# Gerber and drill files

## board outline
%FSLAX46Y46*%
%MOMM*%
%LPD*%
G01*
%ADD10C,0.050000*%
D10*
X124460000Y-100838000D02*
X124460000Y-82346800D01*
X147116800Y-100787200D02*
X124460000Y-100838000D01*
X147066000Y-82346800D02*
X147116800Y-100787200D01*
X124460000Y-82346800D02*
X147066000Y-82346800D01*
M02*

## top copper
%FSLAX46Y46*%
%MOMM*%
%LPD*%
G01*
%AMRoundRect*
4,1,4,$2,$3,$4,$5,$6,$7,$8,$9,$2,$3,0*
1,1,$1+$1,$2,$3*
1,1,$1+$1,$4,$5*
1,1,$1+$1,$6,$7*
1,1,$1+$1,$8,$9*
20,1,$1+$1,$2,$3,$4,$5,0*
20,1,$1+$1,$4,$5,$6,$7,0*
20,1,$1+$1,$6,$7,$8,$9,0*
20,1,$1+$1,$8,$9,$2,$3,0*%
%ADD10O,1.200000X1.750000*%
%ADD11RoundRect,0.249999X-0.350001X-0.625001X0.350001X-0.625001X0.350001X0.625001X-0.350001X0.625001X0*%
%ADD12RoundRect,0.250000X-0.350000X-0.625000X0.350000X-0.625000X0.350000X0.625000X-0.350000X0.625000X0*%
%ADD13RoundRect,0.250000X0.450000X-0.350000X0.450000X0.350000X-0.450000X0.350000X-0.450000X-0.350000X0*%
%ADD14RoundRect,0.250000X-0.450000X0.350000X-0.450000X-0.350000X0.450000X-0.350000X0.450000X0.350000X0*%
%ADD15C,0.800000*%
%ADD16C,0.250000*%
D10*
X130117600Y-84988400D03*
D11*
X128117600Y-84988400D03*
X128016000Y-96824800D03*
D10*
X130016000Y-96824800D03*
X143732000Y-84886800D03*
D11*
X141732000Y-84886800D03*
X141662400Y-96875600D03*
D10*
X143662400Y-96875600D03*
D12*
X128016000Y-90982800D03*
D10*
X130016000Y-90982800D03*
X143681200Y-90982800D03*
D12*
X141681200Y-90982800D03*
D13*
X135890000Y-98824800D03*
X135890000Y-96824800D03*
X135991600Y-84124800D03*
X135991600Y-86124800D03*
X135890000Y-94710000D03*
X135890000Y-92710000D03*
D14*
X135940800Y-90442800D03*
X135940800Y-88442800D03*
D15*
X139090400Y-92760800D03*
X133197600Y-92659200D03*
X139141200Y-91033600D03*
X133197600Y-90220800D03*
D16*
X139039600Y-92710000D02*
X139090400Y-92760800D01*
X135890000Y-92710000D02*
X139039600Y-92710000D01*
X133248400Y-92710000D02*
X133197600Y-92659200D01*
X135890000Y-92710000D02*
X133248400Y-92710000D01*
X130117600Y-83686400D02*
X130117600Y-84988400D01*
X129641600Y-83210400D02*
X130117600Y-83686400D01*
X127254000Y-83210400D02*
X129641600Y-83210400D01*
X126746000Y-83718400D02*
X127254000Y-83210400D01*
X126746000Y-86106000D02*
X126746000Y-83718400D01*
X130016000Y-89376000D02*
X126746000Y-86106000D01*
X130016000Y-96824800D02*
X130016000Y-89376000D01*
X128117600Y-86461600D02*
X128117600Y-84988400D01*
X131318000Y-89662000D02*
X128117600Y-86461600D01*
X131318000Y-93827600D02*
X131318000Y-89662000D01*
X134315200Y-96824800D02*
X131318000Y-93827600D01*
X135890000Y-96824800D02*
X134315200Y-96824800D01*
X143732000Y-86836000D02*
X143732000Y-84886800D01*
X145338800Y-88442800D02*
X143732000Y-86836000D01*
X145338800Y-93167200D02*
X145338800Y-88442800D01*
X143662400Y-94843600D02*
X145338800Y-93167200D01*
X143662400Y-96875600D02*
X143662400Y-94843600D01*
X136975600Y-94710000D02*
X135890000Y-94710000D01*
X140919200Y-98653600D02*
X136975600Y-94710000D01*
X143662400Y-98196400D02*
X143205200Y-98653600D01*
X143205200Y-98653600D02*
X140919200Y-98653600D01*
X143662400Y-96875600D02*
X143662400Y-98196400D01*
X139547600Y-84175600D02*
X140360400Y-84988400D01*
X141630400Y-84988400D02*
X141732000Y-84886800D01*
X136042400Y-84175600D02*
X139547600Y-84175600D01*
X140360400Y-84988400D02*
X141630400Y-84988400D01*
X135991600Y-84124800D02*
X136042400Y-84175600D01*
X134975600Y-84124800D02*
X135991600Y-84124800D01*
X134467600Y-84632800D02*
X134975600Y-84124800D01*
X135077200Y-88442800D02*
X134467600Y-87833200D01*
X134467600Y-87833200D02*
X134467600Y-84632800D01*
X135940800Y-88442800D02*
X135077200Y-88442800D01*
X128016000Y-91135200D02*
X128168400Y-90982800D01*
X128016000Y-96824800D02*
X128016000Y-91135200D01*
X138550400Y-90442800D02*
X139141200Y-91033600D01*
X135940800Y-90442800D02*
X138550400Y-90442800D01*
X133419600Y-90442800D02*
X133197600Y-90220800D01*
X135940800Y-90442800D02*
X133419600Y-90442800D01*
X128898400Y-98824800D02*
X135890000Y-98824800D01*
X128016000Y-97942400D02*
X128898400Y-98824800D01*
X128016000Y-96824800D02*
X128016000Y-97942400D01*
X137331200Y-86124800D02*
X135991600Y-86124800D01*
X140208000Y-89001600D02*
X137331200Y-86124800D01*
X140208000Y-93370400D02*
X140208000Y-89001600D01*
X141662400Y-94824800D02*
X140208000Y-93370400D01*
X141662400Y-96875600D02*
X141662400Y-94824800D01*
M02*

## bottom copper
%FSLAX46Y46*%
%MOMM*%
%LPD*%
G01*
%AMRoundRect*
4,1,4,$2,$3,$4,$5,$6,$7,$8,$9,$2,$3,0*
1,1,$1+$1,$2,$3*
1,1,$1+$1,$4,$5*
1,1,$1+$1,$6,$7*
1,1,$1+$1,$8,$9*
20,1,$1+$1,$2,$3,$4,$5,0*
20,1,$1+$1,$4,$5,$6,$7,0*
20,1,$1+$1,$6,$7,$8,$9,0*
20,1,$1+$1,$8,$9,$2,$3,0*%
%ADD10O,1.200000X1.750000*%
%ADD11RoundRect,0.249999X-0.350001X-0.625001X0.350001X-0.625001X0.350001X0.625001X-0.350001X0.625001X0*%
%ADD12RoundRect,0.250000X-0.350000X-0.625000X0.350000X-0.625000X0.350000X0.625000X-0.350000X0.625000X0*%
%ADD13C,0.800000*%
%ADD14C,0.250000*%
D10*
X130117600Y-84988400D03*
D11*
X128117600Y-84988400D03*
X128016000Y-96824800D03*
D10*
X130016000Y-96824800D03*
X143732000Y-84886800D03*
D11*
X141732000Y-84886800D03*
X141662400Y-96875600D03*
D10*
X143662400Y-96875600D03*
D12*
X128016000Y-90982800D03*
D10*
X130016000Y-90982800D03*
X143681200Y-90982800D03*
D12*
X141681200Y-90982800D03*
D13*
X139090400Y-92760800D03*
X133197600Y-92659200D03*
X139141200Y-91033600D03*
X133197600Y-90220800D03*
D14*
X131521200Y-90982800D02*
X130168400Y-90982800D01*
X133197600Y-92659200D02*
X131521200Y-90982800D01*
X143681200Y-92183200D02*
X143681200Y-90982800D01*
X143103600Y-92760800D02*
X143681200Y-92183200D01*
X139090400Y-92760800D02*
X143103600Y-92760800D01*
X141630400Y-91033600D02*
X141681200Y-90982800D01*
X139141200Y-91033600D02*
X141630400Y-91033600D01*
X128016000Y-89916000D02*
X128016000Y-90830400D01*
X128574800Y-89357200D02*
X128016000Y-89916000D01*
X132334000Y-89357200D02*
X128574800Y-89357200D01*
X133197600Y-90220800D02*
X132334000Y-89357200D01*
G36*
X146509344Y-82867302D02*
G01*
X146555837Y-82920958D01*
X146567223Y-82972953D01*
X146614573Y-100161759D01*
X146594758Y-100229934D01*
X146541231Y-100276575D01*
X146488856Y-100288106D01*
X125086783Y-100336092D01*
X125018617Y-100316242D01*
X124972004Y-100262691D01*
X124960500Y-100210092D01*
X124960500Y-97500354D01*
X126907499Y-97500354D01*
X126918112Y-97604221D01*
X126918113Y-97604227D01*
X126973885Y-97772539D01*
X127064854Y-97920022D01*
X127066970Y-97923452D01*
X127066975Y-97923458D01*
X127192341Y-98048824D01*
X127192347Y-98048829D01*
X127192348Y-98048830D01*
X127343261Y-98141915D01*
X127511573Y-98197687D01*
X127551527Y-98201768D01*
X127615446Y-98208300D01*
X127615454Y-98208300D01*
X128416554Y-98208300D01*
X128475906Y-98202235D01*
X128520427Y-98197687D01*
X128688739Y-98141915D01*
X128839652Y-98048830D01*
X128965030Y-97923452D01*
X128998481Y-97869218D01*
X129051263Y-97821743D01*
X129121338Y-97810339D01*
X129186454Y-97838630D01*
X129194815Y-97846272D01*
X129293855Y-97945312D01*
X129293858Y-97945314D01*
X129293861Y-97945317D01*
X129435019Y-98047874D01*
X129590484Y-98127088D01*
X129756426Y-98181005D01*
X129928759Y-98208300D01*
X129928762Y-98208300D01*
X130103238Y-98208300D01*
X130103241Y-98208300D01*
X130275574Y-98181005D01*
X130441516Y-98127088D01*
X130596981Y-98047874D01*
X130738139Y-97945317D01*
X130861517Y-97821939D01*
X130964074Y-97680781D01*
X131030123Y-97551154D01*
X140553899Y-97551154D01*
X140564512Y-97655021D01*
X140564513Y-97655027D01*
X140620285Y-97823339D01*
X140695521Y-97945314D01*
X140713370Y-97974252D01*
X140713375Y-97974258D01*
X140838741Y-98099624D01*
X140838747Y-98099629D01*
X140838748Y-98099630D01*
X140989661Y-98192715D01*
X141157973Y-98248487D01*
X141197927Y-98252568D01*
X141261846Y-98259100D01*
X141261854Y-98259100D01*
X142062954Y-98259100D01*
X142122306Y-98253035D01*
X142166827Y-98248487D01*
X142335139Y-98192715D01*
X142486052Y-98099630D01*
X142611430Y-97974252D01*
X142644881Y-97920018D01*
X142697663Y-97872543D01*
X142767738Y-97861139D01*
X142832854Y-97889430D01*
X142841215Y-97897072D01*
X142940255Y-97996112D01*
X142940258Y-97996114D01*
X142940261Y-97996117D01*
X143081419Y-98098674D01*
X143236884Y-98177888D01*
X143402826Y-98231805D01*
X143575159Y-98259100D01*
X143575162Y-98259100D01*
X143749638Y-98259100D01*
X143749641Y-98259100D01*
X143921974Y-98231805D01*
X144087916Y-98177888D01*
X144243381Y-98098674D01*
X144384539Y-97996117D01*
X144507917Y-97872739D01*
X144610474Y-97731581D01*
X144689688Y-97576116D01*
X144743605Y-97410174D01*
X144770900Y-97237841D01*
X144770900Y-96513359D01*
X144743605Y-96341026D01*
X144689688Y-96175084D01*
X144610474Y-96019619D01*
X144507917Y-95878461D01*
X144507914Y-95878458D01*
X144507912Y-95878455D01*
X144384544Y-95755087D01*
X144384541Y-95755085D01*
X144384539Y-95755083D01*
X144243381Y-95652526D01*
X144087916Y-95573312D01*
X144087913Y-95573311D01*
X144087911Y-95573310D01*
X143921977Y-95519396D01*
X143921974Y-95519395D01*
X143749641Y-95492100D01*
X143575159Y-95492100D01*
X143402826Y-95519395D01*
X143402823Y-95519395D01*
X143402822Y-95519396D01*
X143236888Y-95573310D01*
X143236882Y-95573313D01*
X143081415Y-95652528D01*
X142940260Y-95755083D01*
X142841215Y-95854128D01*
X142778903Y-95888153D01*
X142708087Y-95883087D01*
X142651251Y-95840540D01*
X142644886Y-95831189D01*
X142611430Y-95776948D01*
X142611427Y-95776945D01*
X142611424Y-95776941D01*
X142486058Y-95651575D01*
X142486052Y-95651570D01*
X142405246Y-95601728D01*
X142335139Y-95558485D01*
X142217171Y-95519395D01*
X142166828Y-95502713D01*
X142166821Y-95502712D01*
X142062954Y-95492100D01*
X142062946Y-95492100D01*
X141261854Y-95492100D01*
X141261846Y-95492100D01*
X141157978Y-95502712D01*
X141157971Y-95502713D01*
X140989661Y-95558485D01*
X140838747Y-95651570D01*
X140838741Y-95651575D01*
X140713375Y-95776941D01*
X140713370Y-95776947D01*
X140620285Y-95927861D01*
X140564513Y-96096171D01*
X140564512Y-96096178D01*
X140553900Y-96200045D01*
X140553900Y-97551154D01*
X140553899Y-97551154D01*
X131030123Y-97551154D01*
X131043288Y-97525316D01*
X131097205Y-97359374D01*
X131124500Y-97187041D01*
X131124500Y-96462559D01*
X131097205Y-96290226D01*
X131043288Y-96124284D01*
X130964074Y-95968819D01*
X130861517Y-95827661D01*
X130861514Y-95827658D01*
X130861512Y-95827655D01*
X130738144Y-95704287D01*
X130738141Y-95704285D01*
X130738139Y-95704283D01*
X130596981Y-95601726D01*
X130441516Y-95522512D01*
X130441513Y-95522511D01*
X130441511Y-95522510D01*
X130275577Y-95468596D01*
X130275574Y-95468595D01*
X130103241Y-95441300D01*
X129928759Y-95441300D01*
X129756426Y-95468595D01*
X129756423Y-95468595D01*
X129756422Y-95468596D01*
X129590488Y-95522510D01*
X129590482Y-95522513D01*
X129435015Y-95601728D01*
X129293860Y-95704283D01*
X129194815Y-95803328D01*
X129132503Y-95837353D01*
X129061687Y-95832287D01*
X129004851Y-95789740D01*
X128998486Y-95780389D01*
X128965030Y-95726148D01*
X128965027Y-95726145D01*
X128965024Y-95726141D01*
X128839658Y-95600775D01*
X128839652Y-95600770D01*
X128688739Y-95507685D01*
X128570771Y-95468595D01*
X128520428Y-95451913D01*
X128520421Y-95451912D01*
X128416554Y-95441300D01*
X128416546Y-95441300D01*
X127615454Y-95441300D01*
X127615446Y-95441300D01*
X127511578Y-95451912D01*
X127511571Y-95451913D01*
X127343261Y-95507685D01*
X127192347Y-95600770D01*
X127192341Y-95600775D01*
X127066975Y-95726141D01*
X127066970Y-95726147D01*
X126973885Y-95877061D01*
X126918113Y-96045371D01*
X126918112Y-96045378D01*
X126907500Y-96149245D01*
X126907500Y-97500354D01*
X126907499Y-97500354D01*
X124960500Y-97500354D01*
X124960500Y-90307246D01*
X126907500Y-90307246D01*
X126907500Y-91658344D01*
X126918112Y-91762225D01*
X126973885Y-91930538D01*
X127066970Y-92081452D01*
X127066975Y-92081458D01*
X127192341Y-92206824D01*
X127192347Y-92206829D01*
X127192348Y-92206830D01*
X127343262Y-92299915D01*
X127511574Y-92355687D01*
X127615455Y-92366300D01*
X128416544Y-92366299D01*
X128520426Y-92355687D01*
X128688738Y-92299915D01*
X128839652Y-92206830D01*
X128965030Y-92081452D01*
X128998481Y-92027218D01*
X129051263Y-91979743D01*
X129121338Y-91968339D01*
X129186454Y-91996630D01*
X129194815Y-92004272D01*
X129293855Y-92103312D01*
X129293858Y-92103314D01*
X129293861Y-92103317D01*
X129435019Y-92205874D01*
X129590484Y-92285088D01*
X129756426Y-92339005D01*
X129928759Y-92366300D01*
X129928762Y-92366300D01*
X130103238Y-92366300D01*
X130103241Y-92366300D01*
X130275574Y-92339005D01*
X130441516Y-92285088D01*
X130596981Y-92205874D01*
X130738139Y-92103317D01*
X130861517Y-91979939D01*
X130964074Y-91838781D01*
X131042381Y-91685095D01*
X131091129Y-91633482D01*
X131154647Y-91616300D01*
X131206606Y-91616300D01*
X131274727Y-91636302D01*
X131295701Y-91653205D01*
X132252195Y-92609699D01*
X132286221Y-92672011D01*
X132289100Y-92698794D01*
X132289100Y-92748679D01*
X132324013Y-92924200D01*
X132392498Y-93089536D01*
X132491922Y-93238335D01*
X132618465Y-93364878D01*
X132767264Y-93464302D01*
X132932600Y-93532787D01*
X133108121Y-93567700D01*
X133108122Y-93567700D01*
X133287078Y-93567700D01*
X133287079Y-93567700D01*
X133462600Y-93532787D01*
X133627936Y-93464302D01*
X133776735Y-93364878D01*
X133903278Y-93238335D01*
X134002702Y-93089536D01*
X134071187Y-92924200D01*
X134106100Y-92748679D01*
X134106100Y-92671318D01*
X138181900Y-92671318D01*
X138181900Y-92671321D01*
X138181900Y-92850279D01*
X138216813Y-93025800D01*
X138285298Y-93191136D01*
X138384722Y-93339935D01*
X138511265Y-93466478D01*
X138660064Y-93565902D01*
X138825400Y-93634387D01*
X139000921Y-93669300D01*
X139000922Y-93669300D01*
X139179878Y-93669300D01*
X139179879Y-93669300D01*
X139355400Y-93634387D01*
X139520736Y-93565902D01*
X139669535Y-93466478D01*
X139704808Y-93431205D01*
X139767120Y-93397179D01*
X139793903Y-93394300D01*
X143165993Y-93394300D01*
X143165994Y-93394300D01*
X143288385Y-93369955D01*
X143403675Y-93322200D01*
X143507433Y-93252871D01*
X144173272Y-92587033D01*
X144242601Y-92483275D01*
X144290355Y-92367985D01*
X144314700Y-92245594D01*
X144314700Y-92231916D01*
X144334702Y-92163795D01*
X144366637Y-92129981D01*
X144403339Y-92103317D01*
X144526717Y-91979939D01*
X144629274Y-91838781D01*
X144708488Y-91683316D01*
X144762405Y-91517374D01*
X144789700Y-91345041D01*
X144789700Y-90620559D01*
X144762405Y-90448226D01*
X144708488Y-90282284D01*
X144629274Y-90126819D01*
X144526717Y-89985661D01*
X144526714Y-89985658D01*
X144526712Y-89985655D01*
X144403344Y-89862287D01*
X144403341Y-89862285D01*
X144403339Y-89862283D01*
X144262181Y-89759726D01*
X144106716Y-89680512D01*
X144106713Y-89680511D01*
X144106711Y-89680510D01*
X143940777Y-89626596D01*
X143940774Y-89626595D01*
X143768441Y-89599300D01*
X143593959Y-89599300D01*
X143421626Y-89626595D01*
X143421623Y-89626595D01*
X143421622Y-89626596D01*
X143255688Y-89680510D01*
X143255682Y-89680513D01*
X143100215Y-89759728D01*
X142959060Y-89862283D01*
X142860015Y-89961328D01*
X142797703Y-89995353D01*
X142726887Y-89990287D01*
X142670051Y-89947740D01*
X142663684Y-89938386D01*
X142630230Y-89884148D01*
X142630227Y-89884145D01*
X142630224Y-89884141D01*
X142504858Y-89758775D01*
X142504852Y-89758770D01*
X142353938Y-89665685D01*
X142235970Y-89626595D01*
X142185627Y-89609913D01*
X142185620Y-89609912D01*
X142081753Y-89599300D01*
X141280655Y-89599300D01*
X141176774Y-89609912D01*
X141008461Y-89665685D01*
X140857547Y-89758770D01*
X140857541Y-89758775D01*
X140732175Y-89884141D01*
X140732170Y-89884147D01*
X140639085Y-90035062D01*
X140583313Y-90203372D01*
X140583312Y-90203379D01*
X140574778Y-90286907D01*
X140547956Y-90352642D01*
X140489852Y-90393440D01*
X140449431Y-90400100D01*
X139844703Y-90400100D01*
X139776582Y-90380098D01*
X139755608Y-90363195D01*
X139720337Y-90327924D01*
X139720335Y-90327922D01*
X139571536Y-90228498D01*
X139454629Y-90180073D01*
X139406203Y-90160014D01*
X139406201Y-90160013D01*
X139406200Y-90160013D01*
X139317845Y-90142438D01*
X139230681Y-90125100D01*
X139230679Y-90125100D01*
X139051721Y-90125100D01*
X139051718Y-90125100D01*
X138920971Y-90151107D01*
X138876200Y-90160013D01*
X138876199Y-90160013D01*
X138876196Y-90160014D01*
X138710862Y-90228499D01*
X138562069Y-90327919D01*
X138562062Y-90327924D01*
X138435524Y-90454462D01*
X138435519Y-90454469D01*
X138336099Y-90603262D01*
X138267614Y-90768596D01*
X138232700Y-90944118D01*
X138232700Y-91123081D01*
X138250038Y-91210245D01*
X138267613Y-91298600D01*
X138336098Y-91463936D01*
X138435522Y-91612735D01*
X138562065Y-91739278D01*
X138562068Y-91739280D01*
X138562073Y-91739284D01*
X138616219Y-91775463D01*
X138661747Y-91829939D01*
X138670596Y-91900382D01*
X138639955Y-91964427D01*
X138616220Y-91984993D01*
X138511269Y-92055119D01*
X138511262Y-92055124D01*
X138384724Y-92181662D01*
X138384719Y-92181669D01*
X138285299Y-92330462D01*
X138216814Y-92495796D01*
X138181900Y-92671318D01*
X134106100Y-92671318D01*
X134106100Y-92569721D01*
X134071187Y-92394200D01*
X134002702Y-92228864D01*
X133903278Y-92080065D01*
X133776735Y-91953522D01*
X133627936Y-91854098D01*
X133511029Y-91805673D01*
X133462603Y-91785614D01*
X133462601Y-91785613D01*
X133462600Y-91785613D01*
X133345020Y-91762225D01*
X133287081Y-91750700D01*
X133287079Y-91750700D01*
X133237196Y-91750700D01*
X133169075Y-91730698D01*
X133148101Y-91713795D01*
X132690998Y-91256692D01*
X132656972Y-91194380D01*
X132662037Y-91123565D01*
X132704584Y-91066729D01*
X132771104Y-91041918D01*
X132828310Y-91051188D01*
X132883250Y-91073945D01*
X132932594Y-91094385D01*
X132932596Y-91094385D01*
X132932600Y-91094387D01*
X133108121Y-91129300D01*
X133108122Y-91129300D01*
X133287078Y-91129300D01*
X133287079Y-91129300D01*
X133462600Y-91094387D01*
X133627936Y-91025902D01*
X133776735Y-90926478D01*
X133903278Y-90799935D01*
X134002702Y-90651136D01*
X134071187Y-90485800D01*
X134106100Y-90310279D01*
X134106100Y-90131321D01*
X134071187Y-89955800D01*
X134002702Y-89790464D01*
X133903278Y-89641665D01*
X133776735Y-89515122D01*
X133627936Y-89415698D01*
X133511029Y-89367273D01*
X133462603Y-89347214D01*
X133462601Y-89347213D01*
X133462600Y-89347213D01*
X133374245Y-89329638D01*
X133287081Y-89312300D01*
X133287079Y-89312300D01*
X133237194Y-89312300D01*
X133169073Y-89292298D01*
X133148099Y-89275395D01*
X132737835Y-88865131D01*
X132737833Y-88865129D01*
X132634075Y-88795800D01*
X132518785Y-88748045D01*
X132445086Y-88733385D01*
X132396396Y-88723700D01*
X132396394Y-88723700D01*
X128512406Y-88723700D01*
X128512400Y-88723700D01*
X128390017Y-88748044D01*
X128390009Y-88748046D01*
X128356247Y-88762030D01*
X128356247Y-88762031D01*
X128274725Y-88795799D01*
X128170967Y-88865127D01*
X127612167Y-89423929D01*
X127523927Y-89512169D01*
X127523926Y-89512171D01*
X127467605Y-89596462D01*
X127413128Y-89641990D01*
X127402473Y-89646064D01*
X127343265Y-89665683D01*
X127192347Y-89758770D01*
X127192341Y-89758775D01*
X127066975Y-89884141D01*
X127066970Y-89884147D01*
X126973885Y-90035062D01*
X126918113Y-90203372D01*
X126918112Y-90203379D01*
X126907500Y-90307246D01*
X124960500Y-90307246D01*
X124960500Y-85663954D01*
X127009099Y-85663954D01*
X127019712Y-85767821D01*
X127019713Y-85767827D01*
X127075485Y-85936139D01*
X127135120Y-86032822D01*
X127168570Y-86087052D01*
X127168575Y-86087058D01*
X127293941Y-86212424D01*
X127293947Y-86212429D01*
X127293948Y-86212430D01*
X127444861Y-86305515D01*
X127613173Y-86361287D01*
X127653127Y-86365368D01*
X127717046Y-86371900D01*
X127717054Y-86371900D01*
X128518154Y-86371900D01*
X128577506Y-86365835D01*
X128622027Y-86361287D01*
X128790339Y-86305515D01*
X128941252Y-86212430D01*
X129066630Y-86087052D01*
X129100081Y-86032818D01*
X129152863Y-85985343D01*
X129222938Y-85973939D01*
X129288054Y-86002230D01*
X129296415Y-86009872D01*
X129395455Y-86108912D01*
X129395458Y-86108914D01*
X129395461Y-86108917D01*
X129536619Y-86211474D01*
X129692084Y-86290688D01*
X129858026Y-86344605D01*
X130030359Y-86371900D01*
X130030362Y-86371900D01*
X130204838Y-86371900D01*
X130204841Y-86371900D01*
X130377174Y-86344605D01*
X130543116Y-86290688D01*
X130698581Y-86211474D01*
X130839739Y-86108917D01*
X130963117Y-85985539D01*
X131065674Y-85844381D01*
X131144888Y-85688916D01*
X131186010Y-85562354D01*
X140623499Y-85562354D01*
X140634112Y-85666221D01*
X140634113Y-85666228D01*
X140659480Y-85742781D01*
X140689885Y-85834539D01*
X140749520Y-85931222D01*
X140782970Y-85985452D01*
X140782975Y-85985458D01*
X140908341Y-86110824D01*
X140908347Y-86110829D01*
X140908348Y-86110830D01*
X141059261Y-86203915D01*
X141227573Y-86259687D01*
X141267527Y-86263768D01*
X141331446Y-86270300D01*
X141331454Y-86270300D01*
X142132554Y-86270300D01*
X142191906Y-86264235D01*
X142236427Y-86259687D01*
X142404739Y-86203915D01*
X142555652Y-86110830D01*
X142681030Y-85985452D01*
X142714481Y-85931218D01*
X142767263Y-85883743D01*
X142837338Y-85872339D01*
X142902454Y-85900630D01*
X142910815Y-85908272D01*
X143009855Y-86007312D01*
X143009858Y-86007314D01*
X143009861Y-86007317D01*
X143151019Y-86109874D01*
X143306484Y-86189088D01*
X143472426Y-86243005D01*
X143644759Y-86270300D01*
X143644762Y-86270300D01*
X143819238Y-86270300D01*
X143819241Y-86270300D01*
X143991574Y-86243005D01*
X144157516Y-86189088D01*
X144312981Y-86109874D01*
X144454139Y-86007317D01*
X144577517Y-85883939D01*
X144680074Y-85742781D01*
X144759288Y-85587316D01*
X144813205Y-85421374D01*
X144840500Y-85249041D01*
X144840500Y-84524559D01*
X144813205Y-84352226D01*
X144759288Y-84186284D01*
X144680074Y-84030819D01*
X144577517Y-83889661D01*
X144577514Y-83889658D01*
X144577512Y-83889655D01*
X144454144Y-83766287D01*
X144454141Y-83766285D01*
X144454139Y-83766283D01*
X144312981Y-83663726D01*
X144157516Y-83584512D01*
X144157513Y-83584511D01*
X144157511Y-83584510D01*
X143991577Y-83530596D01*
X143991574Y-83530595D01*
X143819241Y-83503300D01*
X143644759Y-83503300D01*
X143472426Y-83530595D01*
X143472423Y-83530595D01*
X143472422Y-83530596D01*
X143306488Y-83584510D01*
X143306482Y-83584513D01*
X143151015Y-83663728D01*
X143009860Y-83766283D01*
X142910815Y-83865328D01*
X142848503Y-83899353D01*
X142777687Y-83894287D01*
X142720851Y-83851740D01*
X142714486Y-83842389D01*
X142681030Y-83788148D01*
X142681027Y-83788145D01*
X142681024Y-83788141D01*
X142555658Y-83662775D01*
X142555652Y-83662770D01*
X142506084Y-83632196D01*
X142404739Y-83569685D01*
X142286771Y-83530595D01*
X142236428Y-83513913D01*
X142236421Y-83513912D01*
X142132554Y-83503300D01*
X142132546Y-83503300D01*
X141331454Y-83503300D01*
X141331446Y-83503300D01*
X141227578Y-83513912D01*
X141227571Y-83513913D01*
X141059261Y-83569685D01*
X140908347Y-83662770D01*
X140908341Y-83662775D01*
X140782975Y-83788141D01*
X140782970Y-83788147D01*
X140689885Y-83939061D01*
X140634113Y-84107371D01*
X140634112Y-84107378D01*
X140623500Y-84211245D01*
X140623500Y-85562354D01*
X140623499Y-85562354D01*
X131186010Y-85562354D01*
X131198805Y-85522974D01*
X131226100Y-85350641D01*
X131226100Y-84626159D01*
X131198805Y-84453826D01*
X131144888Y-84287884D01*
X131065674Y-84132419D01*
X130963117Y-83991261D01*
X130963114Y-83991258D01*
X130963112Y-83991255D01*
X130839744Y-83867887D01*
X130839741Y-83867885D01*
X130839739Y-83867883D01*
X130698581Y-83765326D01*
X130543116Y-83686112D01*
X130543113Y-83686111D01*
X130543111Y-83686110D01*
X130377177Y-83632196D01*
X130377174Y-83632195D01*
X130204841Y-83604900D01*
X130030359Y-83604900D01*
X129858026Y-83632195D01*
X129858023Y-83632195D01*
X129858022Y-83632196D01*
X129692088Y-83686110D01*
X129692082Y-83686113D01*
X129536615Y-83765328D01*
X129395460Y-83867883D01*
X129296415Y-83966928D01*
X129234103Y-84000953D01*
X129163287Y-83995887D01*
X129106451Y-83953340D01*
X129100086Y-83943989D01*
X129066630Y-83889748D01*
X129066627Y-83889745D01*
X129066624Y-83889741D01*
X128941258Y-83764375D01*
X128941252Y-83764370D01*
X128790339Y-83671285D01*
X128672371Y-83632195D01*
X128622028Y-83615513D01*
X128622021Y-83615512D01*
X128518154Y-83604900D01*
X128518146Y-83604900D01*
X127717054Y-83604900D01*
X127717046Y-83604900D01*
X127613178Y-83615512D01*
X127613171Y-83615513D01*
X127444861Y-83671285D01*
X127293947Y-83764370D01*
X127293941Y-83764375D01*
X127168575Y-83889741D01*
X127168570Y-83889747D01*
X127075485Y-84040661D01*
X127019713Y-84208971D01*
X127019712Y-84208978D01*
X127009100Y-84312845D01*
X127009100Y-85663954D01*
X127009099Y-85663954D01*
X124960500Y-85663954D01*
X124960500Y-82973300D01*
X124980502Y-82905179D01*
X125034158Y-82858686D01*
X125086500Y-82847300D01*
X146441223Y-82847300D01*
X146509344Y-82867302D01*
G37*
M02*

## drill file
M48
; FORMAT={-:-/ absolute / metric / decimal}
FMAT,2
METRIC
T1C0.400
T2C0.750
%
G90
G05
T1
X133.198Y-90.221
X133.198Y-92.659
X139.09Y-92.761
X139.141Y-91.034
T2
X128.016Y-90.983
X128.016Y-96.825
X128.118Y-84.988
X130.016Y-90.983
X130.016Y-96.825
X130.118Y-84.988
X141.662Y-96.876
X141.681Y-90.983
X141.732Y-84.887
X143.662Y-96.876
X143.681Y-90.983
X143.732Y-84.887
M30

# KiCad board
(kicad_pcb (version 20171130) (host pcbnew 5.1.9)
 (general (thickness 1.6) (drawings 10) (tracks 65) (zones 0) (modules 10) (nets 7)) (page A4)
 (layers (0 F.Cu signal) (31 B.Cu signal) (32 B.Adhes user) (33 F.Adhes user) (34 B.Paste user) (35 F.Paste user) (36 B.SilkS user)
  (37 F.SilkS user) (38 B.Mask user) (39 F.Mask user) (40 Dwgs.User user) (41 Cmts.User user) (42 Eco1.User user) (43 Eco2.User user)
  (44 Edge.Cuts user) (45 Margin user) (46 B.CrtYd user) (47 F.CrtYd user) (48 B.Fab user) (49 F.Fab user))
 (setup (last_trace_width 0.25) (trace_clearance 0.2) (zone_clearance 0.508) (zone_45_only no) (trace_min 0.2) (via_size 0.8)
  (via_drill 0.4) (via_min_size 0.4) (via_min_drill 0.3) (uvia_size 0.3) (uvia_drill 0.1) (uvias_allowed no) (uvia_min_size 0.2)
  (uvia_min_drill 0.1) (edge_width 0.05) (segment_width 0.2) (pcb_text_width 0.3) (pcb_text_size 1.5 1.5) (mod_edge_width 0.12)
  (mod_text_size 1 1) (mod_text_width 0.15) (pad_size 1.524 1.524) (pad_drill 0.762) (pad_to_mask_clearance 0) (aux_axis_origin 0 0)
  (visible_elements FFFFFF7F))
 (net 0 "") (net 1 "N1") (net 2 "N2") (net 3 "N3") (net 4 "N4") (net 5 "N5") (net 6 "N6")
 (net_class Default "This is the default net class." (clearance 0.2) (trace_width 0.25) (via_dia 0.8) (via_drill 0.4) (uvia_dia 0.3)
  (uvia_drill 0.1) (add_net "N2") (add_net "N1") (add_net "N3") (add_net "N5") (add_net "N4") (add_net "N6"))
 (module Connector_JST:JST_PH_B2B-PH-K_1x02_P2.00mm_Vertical (layer F.Cu) (at 128.1176 84.9884)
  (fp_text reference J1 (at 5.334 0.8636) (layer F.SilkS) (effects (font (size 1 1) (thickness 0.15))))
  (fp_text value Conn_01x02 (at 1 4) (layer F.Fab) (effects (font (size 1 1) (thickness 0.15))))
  (pad 2 thru_hole oval (at 2 0) (size 1.2 1.75) (drill 0.75) (layers *.Cu *.Mask) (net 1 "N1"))
  (pad 1 thru_hole roundrect (at 0 0) (size 1.2 1.75) (drill 0.75) (layers *.Cu *.Mask) (roundrect_rratio 0.2083325) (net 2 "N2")))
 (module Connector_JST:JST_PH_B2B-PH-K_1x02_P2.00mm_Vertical (layer F.Cu) (at 128.016 96.8248)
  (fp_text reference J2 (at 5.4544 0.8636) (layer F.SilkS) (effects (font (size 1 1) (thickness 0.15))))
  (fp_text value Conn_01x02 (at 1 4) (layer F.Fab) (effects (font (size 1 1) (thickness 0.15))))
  (pad 1 thru_hole roundrect (at 0 0) (size 1.2 1.75) (drill 0.75) (layers *.Cu *.Mask) (roundrect_rratio 0.2083325) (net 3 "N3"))
  (pad 2 thru_hole oval (at 2 0) (size 1.2 1.75) (drill 0.75) (layers *.Cu *.Mask) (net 1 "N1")))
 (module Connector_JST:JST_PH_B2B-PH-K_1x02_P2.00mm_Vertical (layer F.Cu) (at 141.732 84.8868)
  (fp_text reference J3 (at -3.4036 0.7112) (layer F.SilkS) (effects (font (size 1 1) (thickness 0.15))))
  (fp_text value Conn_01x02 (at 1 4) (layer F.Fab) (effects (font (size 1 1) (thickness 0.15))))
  (pad 2 thru_hole oval (at 2 0) (size 1.2 1.75) (drill 0.75) (layers *.Cu *.Mask) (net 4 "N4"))
  (pad 1 thru_hole roundrect (at 0 0) (size 1.2 1.75) (drill 0.75) (layers *.Cu *.Mask) (roundrect_rratio 0.2083325) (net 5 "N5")))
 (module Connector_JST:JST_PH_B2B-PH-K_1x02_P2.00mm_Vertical (layer F.Cu) (at 141.6624 96.8756)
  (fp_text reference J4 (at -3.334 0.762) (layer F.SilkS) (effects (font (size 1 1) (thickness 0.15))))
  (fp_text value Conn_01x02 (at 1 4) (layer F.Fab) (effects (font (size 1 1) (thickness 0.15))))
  (pad 1 thru_hole roundrect (at 0 0) (size 1.2 1.75) (drill 0.75) (layers *.Cu *.Mask) (roundrect_rratio 0.2083325) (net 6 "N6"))
  (pad 2 thru_hole oval (at 2 0) (size 1.2 1.75) (drill 0.75) (layers *.Cu *.Mask) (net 4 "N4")))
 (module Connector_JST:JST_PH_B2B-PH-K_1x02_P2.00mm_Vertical (layer F.Cu) (at 128.016 90.9828)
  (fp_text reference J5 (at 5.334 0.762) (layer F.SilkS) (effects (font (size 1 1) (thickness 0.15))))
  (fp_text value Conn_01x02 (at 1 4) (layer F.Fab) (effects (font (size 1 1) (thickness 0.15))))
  (pad 1 thru_hole roundrect (at 0 0) (size 1.2 1.75) (drill 0.75) (layers *.Cu *.Mask) (roundrect_rratio 0.208333) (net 3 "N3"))
  (pad 2 thru_hole oval (at 2 0) (size 1.2 1.75) (drill 0.75) (layers *.Cu *.Mask) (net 1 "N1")))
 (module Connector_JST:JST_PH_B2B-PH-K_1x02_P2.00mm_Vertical (layer F.Cu) (at 141.6812 90.9828)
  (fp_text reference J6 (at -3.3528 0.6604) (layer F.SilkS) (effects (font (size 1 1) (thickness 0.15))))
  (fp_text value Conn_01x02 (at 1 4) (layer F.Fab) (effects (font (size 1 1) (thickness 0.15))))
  (pad 2 thru_hole oval (at 2 0) (size 1.2 1.75) (drill 0.75) (layers *.Cu *.Mask) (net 1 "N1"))
  (pad 1 thru_hole roundrect (at 0 0) (size 1.2 1.75) (drill 0.75) (layers *.Cu *.Mask) (roundrect_rratio 0.208333) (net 3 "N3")))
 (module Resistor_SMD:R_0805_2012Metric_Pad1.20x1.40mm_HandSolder (layer F.Cu) (at 135.89 97.8248 90)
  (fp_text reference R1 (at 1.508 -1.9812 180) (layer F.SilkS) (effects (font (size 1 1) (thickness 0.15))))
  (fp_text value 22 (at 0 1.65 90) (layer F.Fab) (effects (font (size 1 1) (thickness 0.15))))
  (pad 1 smd roundrect (at -1 0 90) (size 1.2 1.4) (layers F.Cu F.Paste F.Mask) (roundrect_rratio 0.208333) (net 3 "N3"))
  (pad 2 smd roundrect (at 1 0 90) (size 1.2 1.4) (layers F.Cu F.Paste F.Mask) (roundrect_rratio 0.208333) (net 2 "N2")))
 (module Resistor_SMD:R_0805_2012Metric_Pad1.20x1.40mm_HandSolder (layer F.Cu) (at 135.9916 85.1248 90)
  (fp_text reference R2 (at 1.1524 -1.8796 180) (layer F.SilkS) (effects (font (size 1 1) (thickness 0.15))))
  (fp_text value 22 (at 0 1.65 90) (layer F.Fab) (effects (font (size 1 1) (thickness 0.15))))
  (pad 2 smd roundrect (at 1 0 90) (size 1.2 1.4) (layers F.Cu F.Paste F.Mask) (roundrect_rratio 0.208333) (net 5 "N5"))
  (pad 1 smd roundrect (at -1 0 90) (size 1.2 1.4) (layers F.Cu F.Paste F.Mask) (roundrect_rratio 0.208333) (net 6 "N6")))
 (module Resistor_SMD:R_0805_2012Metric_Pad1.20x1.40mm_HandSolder (layer F.Cu) (at 135.89 93.71 90)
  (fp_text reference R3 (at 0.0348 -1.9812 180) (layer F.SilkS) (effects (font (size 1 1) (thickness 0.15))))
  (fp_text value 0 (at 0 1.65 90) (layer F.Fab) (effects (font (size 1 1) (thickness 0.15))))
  (pad 1 smd roundrect (at -1 0 90) (size 1.2 1.4) (layers F.Cu F.Paste F.Mask) (roundrect_rratio 0.208333) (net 4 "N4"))
  (pad 2 smd roundrect (at 1 0 90) (size 1.2 1.4) (layers F.Cu F.Paste F.Mask) (roundrect_rratio 0.208333) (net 1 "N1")))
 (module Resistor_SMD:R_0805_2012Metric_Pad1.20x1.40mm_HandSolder (layer F.Cu) (at 135.9408 89.4428 270)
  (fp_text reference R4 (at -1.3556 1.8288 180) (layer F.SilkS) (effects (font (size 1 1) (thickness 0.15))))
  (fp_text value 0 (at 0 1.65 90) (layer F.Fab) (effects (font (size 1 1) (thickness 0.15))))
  (pad 2 smd roundrect (at 1 0 270) (size 1.2 1.4) (layers F.Cu F.Paste F.Mask) (roundrect_rratio 0.208333) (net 3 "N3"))
  (pad 1 smd roundrect (at -1 0 270) (size 1.2 1.4) (layers F.Cu F.Paste F.Mask) (roundrect_rratio 0.208333) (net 5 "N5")))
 (gr_line (start 124.46 100.838) (end 124.46 82.3468) (layer Edge.Cuts) (width 0.05))
 (gr_line (start 147.1168 100.7872) (end 124.46 100.838) (layer Edge.Cuts) (width 0.05))
 (gr_line (start 147.066 82.3468) (end 147.1168 100.7872) (layer Edge.Cuts) (width 0.05))
 (gr_line (start 124.46 82.3468) (end 147.066 82.3468) (layer Edge.Cuts) (width 0.05))
 (via (at 139.0904 92.7608) (size 0.8) (drill 0.4) (layers F.Cu B.Cu) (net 1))
 (segment (start 139.0396 92.71) (end 139.0904 92.7608) (width 0.25) (layer F.Cu) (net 1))
 (segment (start 135.89 92.71) (end 139.0396 92.71) (width 0.25) (layer F.Cu) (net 1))
 (via (at 133.1976 92.6592) (size 0.8) (drill 0.4) (layers F.Cu B.Cu) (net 1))
 (segment (start 133.2484 92.71) (end 133.1976 92.6592) (width 0.25) (layer F.Cu) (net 1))
 (segment (start 135.89 92.71) (end 133.2484 92.71) (width 0.25) (layer F.Cu) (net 1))
 (segment (start 131.5212 90.9828) (end 130.1684 90.9828) (width 0.25) (layer B.Cu) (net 1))
 (segment (start 133.1976 92.6592) (end 131.5212 90.9828) (width 0.25) (layer B.Cu) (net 1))
 (segment (start 130.1176 83.6864) (end 130.1176 84.9884) (width 0.25) (layer F.Cu) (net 1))
 (segment (start 129.6416 83.2104) (end 130.1176 83.6864) (width 0.25) (layer F.Cu) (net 1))
 (segment (start 127.254 83.2104) (end 129.6416 83.2104) (width 0.25) (layer F.Cu) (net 1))
 (segment (start 126.746 83.7184) (end 127.254 83.2104) (width 0.25) (layer F.Cu) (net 1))
 (segment (start 126.746 86.106) (end 126.746 83.7184) (width 0.25) (layer F.Cu) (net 1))
 (segment (start 130.016 89.376) (end 126.746 86.106) (width 0.25) (layer F.Cu) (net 1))
 (segment (start 130.016 96.8248) (end 130.016 89.376) (width 0.25) (layer F.Cu) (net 1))
 (segment (start 143.6812 92.1832) (end 143.6812 90.9828) (width 0.25) (layer B.Cu) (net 1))
 (segment (start 143.1036 92.7608) (end 143.6812 92.1832) (width 0.25) (layer B.Cu) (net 1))
 (segment (start 139.0904 92.7608) (end 143.1036 92.7608) (width 0.25) (layer B.Cu) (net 1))
 (segment (start 128.1176 86.4616) (end 128.1176 84.9884) (width 0.25) (layer F.Cu) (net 2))
 (segment (start 131.318 89.662) (end 128.1176 86.4616) (width 0.25) (layer F.Cu) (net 2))
 (segment (start 131.318 93.8276) (end 131.318 89.662) (width 0.25) (layer F.Cu) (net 2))
 (segment (start 134.3152 96.8248) (end 131.318 93.8276) (width 0.25) (layer F.Cu) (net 2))
 (segment (start 135.89 96.8248) (end 134.3152 96.8248) (width 0.25) (layer F.Cu) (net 2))
 (segment (start 143.732 86.836) (end 143.732 84.8868) (width 0.25) (layer F.Cu) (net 4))
 (segment (start 145.3388 88.4428) (end 143.732 86.836) (width 0.25) (layer F.Cu) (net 4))
 (segment (start 145.3388 93.1672) (end 145.3388 88.4428) (width 0.25) (layer F.Cu) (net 4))
 (segment (start 143.6624 94.8436) (end 145.3388 93.1672) (width 0.25) (layer F.Cu) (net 4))
 (segment (start 143.6624 96.8756) (end 143.6624 94.8436) (width 0.25) (layer F.Cu) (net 4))
 (segment (start 136.9756 94.71) (end 135.89 94.71) (width 0.25) (layer F.Cu) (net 4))
 (segment (start 140.9192 98.6536) (end 136.9756 94.71) (width 0.25) (layer F.Cu) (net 4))
 (segment (start 143.6624 98.1964) (end 143.2052 98.6536) (width 0.25) (layer F.Cu) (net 4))
 (segment (start 143.2052 98.6536) (end 140.9192 98.6536) (width 0.25) (layer F.Cu) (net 4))
 (segment (start 143.6624 96.8756) (end 143.6624 98.1964) (width 0.25) (layer F.Cu) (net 4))
 (segment (start 139.5476 84.1756) (end 140.3604 84.9884) (width 0.25) (layer F.Cu) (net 5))
 (segment (start 141.6304 84.9884) (end 141.732 84.8868) (width 0.25) (layer F.Cu) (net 5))
 (segment (start 136.0424 84.1756) (end 139.5476 84.1756) (width 0.25) (layer F.Cu) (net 5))
 (segment (start 140.3604 84.9884) (end 141.6304 84.9884) (width 0.25) (layer F.Cu) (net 5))
 (segment (start 135.9916 84.1248) (end 136.0424 84.1756) (width 0.25) (layer F.Cu) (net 5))
 (segment (start 134.9756 84.1248) (end 135.9916 84.1248) (width 0.25) (layer F.Cu) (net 5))
 (segment (start 134.4676 84.6328) (end 134.9756 84.1248) (width 0.25) (layer F.Cu) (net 5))
 (segment (start 135.0772 88.4428) (end 134.4676 87.8332) (width 0.25) (layer F.Cu) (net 5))
 (segment (start 134.4676 87.8332) (end 134.4676 84.6328) (width 0.25) (layer F.Cu) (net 5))
 (segment (start 135.9408 88.4428) (end 135.0772 88.4428) (width 0.25) (layer F.Cu) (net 5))
 (segment (start 128.016 91.1352) (end 128.1684 90.9828) (width 0.25) (layer F.Cu) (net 3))
 (segment (start 128.016 96.8248) (end 128.016 91.1352) (width 0.25) (layer F.Cu) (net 3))
 (via (at 139.1412 91.0336) (size 0.8) (drill 0.4) (layers F.Cu B.Cu) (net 3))
 (segment (start 138.5504 90.4428) (end 139.1412 91.0336) (width 0.25) (layer F.Cu) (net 3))
 (segment (start 135.9408 90.4428) (end 138.5504 90.4428) (width 0.25) (layer F.Cu) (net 3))
 (segment (start 141.6304 91.0336) (end 141.6812 90.9828) (width 0.25) (layer B.Cu) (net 3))
 (segment (start 139.1412 91.0336) (end 141.6304 91.0336) (width 0.25) (layer B.Cu) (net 3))
 (via (at 133.1976 90.2208) (size 0.8) (drill 0.4) (layers F.Cu B.Cu) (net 3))
 (segment (start 133.4196 90.4428) (end 133.1976 90.2208) (width 0.25) (layer F.Cu) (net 3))
 (segment (start 135.9408 90.4428) (end 133.4196 90.4428) (width 0.25) (layer F.Cu) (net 3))
 (segment (start 128.8984 98.8248) (end 135.89 98.8248) (width 0.25) (layer F.Cu) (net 3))
 (segment (start 128.016 97.9424) (end 128.8984 98.8248) (width 0.25) (layer F.Cu) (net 3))
 (segment (start 128.016 96.8248) (end 128.016 97.9424) (width 0.25) (layer F.Cu) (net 3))
 (segment (start 128.016 89.916) (end 128.016 90.8304) (width 0.25) (layer B.Cu) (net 3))
 (segment (start 128.5748 89.3572) (end 128.016 89.916) (width 0.25) (layer B.Cu) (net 3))
 (segment (start 132.334 89.3572) (end 128.5748 89.3572) (width 0.25) (layer B.Cu) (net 3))
 (segment (start 133.1976 90.2208) (end 132.334 89.3572) (width 0.25) (layer B.Cu) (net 3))
 (segment (start 137.3312 86.1248) (end 135.9916 86.1248) (width 0.25) (layer F.Cu) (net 6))
 (segment (start 140.208 89.0016) (end 137.3312 86.1248) (width 0.25) (layer F.Cu) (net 6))
 (segment (start 140.208 93.3704) (end 140.208 89.0016) (width 0.25) (layer F.Cu) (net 6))
 (segment (start 141.6624 94.8248) (end 140.208 93.3704) (width 0.25) (layer F.Cu) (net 6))
 (segment (start 141.6624 96.8756) (end 141.6624 94.8248) (width 0.25) (layer F.Cu) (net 6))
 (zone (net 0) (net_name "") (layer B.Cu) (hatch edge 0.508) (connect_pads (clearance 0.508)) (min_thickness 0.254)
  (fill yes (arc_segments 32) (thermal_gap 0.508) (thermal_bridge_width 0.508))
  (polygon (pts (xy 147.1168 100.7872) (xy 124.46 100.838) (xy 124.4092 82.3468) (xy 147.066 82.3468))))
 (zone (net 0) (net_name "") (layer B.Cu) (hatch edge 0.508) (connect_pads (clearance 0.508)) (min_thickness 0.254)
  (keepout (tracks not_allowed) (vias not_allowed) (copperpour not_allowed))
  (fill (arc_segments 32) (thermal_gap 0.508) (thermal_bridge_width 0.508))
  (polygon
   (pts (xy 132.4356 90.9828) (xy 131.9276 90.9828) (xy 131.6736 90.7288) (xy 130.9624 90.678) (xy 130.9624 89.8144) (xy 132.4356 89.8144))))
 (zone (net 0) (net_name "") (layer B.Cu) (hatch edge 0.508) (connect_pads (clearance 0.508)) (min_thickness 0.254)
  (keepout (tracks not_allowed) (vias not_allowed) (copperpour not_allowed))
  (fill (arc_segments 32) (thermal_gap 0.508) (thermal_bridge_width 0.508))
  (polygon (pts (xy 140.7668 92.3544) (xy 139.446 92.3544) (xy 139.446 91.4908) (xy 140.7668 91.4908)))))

